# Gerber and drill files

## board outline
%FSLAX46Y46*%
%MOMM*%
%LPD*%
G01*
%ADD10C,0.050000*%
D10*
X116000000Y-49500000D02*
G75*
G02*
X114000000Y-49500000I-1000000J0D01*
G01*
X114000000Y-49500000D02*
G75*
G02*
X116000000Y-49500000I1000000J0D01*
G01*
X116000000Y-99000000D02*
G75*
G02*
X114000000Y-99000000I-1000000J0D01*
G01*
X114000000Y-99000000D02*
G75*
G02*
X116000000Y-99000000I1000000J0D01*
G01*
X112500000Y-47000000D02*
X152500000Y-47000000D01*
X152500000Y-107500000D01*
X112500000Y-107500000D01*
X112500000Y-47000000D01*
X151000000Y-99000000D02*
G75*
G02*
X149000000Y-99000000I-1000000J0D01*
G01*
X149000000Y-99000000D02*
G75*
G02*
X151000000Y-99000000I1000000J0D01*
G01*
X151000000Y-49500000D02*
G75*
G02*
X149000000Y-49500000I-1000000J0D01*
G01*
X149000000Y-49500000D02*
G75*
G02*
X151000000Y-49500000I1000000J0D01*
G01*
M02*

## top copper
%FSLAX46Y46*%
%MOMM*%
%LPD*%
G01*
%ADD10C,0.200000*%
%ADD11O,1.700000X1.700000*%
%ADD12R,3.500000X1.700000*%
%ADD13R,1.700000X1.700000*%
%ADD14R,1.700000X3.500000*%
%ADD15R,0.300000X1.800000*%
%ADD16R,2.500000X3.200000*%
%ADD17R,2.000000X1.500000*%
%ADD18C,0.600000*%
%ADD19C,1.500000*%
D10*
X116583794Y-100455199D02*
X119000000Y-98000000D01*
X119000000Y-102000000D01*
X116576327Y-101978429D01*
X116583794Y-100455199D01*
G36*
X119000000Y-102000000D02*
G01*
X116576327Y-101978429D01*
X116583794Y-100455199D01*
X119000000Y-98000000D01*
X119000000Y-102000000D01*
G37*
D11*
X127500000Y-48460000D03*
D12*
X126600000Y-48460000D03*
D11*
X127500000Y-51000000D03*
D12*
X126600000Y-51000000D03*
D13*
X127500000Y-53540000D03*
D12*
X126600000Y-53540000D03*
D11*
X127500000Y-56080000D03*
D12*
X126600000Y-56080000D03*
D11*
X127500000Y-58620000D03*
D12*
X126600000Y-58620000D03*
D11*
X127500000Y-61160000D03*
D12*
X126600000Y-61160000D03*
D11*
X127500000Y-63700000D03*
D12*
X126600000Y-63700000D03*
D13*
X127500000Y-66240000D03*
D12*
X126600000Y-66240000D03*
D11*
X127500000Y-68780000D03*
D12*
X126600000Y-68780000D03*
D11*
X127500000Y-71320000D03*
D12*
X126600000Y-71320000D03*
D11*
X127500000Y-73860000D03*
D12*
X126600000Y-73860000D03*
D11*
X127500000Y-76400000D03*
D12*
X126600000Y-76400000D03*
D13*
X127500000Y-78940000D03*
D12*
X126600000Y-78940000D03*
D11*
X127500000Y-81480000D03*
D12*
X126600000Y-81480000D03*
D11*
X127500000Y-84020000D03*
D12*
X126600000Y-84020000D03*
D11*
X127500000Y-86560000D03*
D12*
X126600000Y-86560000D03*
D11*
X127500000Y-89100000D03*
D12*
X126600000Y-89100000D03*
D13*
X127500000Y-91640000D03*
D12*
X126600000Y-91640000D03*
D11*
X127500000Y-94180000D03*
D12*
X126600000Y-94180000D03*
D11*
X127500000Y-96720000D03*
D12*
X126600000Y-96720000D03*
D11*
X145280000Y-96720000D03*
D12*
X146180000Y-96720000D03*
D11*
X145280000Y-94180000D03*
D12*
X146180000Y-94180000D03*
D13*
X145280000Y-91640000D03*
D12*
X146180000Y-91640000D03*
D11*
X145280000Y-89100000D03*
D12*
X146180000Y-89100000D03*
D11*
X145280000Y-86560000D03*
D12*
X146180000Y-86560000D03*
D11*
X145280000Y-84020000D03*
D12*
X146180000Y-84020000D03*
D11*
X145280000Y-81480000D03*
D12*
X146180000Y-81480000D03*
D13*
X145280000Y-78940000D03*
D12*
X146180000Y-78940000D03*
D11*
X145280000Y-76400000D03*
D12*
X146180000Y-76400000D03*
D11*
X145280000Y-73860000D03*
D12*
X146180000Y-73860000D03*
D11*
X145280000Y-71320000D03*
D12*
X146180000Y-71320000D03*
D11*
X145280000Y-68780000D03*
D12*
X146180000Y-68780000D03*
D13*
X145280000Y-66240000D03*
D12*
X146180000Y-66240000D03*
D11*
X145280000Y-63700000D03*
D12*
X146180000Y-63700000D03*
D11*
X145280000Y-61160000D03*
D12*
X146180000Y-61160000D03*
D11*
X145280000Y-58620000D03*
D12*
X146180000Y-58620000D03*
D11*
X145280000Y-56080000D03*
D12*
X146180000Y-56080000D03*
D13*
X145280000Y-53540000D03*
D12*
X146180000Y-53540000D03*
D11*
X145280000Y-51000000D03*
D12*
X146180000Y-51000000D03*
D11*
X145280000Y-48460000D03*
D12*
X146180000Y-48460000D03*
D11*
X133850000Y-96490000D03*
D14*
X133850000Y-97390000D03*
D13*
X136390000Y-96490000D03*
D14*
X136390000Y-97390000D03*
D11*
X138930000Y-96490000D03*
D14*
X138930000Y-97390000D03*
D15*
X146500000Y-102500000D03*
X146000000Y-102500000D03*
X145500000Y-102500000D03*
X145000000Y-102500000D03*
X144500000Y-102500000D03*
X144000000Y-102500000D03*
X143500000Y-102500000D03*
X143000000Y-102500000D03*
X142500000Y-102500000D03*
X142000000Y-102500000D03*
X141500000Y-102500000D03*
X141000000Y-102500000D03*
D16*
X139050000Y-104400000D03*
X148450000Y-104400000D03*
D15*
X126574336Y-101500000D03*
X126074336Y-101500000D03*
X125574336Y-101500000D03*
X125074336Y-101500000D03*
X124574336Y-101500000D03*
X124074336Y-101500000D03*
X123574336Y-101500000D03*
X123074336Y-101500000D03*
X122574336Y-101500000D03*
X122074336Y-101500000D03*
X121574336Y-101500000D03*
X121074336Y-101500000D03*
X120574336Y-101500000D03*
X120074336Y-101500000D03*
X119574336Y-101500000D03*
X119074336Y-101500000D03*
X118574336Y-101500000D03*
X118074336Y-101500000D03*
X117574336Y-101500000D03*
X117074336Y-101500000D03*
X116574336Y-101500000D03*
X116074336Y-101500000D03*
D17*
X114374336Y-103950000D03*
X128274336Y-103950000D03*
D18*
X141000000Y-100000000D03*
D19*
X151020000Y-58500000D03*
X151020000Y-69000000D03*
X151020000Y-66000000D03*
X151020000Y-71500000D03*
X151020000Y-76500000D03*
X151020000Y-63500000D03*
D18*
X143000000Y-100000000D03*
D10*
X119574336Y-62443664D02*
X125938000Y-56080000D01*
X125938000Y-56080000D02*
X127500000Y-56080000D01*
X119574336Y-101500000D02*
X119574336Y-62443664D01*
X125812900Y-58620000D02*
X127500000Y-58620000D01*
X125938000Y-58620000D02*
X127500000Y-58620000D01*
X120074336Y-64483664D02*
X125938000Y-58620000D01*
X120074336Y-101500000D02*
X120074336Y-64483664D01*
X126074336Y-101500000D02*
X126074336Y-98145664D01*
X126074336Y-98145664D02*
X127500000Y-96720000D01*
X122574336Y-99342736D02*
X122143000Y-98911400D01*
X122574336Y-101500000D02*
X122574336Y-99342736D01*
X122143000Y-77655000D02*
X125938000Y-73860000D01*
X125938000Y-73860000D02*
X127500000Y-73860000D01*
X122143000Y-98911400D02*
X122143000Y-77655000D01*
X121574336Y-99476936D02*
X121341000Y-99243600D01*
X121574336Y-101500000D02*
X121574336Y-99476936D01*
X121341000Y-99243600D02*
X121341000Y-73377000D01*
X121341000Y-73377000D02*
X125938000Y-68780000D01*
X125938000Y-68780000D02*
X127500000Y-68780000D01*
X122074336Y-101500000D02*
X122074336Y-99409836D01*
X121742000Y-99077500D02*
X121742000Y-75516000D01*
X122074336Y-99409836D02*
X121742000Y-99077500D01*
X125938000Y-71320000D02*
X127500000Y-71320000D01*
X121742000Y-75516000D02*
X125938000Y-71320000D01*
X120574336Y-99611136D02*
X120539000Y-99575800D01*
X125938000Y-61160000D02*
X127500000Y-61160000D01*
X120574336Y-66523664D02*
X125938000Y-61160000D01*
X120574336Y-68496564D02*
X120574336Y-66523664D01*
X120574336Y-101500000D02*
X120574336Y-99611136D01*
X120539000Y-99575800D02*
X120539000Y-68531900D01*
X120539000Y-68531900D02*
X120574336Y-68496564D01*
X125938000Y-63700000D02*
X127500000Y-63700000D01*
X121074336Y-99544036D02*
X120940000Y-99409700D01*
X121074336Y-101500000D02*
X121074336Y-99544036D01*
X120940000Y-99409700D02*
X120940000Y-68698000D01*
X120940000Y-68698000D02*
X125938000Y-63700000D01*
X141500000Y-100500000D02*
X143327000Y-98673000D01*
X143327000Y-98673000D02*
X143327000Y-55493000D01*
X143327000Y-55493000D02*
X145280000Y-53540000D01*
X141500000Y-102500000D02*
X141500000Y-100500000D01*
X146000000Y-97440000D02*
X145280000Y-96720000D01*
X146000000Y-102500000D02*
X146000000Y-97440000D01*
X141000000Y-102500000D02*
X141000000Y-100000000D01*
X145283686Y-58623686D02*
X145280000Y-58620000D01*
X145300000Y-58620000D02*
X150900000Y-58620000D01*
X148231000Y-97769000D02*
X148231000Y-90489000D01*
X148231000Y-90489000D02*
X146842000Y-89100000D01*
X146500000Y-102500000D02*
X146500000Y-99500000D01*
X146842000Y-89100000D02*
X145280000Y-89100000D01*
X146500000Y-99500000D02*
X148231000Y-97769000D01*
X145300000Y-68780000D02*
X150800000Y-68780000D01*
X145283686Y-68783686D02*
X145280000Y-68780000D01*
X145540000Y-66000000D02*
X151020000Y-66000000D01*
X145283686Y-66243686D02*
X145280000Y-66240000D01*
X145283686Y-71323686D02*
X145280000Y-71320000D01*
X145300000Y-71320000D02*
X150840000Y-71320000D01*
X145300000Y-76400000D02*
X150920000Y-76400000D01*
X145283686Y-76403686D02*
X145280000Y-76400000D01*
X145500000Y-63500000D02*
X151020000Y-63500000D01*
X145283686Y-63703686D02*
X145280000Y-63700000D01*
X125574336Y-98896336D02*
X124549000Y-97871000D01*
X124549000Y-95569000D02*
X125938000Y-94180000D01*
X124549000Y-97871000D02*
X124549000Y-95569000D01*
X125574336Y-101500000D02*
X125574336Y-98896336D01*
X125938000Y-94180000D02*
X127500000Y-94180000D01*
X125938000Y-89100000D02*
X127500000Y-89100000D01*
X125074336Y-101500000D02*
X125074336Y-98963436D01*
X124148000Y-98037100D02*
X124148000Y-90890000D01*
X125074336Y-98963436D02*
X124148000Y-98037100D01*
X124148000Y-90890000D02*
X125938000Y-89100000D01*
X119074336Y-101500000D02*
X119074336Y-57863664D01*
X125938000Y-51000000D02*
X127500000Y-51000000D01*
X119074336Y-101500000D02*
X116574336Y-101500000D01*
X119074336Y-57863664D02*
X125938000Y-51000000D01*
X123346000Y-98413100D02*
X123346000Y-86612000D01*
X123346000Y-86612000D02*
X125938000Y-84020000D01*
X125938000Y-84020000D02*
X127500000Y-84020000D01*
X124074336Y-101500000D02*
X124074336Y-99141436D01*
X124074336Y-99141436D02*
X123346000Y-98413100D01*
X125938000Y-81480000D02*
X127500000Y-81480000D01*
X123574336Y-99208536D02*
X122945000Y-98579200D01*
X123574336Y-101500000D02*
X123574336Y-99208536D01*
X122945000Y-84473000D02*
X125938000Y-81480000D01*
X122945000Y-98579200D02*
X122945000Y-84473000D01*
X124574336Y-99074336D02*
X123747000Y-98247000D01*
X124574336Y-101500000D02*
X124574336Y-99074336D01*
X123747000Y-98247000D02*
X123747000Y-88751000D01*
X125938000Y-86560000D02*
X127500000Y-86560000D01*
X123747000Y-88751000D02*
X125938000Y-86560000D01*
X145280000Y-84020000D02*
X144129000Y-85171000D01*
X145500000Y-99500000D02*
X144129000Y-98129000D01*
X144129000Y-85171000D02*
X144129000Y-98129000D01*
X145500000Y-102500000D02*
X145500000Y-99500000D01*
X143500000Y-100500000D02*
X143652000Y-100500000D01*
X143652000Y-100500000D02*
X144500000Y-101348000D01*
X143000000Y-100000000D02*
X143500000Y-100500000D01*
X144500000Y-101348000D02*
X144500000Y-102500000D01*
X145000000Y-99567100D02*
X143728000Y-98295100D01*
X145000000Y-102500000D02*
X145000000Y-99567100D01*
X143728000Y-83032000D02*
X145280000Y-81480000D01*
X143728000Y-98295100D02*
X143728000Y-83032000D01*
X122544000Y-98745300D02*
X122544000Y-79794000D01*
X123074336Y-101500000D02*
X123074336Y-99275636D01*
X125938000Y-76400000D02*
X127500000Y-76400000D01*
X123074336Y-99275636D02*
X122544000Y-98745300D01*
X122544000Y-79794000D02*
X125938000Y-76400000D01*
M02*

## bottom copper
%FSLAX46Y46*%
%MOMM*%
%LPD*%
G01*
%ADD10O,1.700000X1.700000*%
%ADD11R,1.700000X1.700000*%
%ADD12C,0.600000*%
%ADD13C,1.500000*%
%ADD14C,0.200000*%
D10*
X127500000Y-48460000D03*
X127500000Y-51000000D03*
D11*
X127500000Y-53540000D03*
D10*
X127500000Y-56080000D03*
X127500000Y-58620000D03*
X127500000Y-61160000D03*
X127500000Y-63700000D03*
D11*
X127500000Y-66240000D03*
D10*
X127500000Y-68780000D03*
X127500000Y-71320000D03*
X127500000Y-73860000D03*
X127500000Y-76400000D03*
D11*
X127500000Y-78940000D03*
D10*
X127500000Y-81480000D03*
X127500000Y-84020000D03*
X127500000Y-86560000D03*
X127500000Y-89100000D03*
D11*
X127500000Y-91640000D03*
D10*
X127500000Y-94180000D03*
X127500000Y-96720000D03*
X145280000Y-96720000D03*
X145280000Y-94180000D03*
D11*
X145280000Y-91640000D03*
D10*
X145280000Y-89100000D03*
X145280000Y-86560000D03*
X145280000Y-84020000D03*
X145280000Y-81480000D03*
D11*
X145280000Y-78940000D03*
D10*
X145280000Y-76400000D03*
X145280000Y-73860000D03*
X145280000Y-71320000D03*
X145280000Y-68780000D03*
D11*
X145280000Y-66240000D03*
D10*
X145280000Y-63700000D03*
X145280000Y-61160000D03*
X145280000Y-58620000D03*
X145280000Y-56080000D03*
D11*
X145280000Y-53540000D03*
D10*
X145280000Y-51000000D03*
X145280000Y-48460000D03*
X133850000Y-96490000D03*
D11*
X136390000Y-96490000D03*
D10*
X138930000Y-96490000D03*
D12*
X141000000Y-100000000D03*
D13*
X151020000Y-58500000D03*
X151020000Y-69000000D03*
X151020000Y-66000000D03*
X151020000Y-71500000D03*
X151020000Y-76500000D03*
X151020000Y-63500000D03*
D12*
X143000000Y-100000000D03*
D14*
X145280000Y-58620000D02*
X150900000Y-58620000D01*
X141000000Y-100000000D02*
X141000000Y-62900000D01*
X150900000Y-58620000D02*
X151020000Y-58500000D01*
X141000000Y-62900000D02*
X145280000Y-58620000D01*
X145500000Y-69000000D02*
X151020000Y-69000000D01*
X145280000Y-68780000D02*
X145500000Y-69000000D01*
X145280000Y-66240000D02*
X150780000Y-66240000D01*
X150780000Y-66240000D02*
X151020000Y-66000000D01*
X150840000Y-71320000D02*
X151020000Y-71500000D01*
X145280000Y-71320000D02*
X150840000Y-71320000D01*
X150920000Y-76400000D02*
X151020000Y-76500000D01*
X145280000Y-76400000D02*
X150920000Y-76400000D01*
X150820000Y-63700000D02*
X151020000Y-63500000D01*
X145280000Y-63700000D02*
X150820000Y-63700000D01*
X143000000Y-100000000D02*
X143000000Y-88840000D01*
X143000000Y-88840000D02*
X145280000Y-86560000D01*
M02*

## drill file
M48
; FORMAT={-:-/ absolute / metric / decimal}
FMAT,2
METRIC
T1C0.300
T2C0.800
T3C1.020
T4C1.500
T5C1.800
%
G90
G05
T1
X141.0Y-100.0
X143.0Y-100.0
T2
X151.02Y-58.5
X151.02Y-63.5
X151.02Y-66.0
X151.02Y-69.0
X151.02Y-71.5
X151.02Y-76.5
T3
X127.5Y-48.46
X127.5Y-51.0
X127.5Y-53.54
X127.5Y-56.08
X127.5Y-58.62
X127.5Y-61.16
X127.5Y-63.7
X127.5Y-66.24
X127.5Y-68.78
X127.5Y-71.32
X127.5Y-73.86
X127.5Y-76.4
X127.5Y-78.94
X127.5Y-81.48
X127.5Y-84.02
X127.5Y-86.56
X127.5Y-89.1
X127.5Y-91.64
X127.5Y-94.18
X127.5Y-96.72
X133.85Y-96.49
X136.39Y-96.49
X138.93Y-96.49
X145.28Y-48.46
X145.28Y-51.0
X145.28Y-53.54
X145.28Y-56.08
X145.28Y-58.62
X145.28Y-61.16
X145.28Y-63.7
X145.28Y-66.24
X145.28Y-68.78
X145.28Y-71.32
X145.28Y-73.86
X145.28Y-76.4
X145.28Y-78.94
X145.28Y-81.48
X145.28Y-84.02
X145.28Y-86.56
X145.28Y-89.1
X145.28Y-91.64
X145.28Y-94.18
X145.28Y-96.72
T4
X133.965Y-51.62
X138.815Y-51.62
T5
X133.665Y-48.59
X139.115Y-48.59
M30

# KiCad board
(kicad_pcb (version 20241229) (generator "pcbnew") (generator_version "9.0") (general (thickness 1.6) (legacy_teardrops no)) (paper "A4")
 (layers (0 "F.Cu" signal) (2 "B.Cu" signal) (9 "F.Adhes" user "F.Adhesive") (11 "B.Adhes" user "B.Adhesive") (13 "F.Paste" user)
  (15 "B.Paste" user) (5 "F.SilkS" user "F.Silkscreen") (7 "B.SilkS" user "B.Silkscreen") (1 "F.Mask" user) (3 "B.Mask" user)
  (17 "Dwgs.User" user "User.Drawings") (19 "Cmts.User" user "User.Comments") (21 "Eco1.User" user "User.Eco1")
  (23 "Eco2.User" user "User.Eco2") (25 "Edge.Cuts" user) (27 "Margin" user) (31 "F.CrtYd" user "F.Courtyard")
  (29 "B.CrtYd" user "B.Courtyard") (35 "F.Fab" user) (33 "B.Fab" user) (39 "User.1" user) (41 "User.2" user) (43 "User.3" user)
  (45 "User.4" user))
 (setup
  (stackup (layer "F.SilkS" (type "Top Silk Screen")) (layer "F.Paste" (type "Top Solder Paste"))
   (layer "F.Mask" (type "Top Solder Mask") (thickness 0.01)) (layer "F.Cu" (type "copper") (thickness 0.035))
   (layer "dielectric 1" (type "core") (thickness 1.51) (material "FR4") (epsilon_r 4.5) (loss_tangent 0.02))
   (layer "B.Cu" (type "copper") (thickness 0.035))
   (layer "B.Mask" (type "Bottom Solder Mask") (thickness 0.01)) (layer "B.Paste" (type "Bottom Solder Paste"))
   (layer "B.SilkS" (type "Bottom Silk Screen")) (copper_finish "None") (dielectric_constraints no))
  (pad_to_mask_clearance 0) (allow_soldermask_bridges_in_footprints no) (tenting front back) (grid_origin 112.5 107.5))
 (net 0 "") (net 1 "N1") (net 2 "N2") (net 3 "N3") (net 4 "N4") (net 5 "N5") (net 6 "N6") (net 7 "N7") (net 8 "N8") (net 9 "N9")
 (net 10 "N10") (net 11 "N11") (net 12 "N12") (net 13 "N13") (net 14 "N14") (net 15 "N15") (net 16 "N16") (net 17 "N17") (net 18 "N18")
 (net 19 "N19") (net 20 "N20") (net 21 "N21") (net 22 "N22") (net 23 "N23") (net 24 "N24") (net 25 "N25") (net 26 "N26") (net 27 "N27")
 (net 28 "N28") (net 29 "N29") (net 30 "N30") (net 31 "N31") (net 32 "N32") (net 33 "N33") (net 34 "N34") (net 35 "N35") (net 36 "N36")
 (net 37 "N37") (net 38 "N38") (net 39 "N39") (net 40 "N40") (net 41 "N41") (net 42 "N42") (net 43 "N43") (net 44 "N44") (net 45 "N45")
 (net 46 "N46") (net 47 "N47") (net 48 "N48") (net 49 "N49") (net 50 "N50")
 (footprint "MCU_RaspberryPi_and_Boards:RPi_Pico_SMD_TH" (layer "F.Cu") (at 136.39 72.59)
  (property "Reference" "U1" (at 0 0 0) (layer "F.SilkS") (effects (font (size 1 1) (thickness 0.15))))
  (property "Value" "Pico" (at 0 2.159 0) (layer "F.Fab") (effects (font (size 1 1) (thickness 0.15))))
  (pad "" np_thru_hole oval (at -2.725 -24) (size 1.8 1.8) (drill 1.8) (layers "*.Cu" "*.Mask"))
  (pad "" np_thru_hole oval (at -2.425 -20.97) (size 1.5 1.5) (drill 1.5) (layers "*.Cu" "*.Mask"))
  (pad "" np_thru_hole oval (at 2.425 -20.97) (size 1.5 1.5) (drill 1.5) (layers "*.Cu" "*.Mask"))
  (pad "" np_thru_hole oval (at 2.725 -24) (size 1.8 1.8) (drill 1.8) (layers "*.Cu" "*.Mask"))
  (pad "1" thru_hole oval (at -8.89 -24.13) (size 1.7 1.7) (drill 1.02) (layers "*.Cu" "*.Mask") (remove_unused_layers no) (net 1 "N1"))
  (pad "1" smd rect (at -8.89 -24.13) (size 3.5 1.7) (drill (offset -0.9 0)) (layers "F.Cu" "F.Mask") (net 1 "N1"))
  (pad "2" thru_hole oval (at -8.89 -21.59) (size 1.7 1.7) (drill 1.02) (layers "*.Cu" "*.Mask") (remove_unused_layers no) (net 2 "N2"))
  (pad "2" smd rect (at -8.89 -21.59) (size 3.5 1.7) (drill (offset -0.9 0)) (layers "F.Cu" "F.Mask") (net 2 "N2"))
  (pad "3" thru_hole rect (at -8.89 -19.05) (size 1.7 1.7) (drill 1.02) (layers "*.Cu" "*.Mask") (remove_unused_layers no) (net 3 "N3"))
  (pad "3" smd rect (at -8.89 -19.05) (size 3.5 1.7) (drill (offset -0.9 0)) (layers "F.Cu" "F.Mask") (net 3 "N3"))
  (pad "4" thru_hole oval (at -8.89 -16.51) (size 1.7 1.7) (drill 1.02) (layers "*.Cu" "*.Mask") (remove_unused_layers no) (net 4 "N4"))
  (pad "4" smd rect (at -8.89 -16.51) (size 3.5 1.7) (drill (offset -0.9 0)) (layers "F.Cu" "F.Mask") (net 4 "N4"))
  (pad "5" thru_hole oval (at -8.89 -13.97) (size 1.7 1.7) (drill 1.02) (layers "*.Cu" "*.Mask") (remove_unused_layers no) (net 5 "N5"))
  (pad "5" smd rect (at -8.89 -13.97) (size 3.5 1.7) (drill (offset -0.9 0)) (layers "F.Cu" "F.Mask") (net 5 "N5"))
  (pad "6" thru_hole oval (at -8.89 -11.43) (size 1.7 1.7) (drill 1.02) (layers "*.Cu" "*.Mask") (remove_unused_layers no) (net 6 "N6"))
  (pad "6" smd rect (at -8.89 -11.43) (size 3.5 1.7) (drill (offset -0.9 0)) (layers "F.Cu" "F.Mask") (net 6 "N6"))
  (pad "7" thru_hole oval (at -8.89 -8.89) (size 1.7 1.7) (drill 1.02) (layers "*.Cu" "*.Mask") (remove_unused_layers no) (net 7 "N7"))
  (pad "7" smd rect (at -8.89 -8.89) (size 3.5 1.7) (drill (offset -0.9 0)) (layers "F.Cu" "F.Mask") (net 7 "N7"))
  (pad "8" thru_hole rect (at -8.89 -6.35) (size 1.7 1.7) (drill 1.02) (layers "*.Cu" "*.Mask") (remove_unused_layers no) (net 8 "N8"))
  (pad "8" smd rect (at -8.89 -6.35) (size 3.5 1.7) (drill (offset -0.9 0)) (layers "F.Cu" "F.Mask") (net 8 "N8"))
  (pad "9" thru_hole oval (at -8.89 -3.81) (size 1.7 1.7) (drill 1.02) (layers "*.Cu" "*.Mask") (remove_unused_layers no) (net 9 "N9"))
  (pad "9" smd rect (at -8.89 -3.81) (size 3.5 1.7) (drill (offset -0.9 0)) (layers "F.Cu" "F.Mask") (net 9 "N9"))
  (pad "10" thru_hole oval (at -8.89 -1.27) (size 1.7 1.7) (drill 1.02) (layers "*.Cu" "*.Mask") (remove_unused_layers no) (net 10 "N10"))
  (pad "10" smd rect (at -8.89 -1.27) (size 3.5 1.7) (drill (offset -0.9 0)) (layers "F.Cu" "F.Mask") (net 10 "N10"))
  (pad "11" thru_hole oval (at -8.89 1.27) (size 1.7 1.7) (drill 1.02) (layers "*.Cu" "*.Mask") (remove_unused_layers no) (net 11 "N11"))
  (pad "11" smd rect (at -8.89 1.27) (size 3.5 1.7) (drill (offset -0.9 0)) (layers "F.Cu" "F.Mask") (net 11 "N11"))
  (pad "12" thru_hole oval (at -8.89 3.81) (size 1.7 1.7) (drill 1.02) (layers "*.Cu" "*.Mask") (remove_unused_layers no) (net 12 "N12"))
  (pad "12" smd rect (at -8.89 3.81) (size 3.5 1.7) (drill (offset -0.9 0)) (layers "F.Cu" "F.Mask") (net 12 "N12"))
  (pad "13" thru_hole rect (at -8.89 6.35) (size 1.7 1.7) (drill 1.02) (layers "*.Cu" "*.Mask") (remove_unused_layers no) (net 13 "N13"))
  (pad "13" smd rect (at -8.89 6.35) (size 3.5 1.7) (drill (offset -0.9 0)) (layers "F.Cu" "F.Mask") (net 13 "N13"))
  (pad "14" thru_hole oval (at -8.89 8.89) (size 1.7 1.7) (drill 1.02) (layers "*.Cu" "*.Mask") (remove_unused_layers no) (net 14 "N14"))
  (pad "14" smd rect (at -8.89 8.89) (size 3.5 1.7) (drill (offset -0.9 0)) (layers "F.Cu" "F.Mask") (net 14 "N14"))
  (pad "15" thru_hole oval (at -8.89 11.43) (size 1.7 1.7) (drill 1.02) (layers "*.Cu" "*.Mask") (remove_unused_layers no) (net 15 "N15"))
  (pad "15" smd rect (at -8.89 11.43) (size 3.5 1.7) (drill (offset -0.9 0)) (layers "F.Cu" "F.Mask") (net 15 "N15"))
  (pad "16" thru_hole oval (at -8.89 13.97) (size 1.7 1.7) (drill 1.02) (layers "*.Cu" "*.Mask") (remove_unused_layers no) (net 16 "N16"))
  (pad "16" smd rect (at -8.89 13.97) (size 3.5 1.7) (drill (offset -0.9 0)) (layers "F.Cu" "F.Mask") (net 16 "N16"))
  (pad "17" thru_hole oval (at -8.89 16.51) (size 1.7 1.7) (drill 1.02) (layers "*.Cu" "*.Mask") (remove_unused_layers no) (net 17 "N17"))
  (pad "17" smd rect (at -8.89 16.51) (size 3.5 1.7) (drill (offset -0.9 0)) (layers "F.Cu" "F.Mask") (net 17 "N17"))
  (pad "18" thru_hole rect (at -8.89 19.05) (size 1.7 1.7) (drill 1.02) (layers "*.Cu" "*.Mask") (remove_unused_layers no) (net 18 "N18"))
  (pad "18" smd rect (at -8.89 19.05) (size 3.5 1.7) (drill (offset -0.9 0)) (layers "F.Cu" "F.Mask") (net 18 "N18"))
  (pad "19" thru_hole oval (at -8.89 21.59) (size 1.7 1.7) (drill 1.02) (layers "*.Cu" "*.Mask") (remove_unused_layers no) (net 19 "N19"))
  (pad "19" smd rect (at -8.89 21.59) (size 3.5 1.7) (drill (offset -0.9 0)) (layers "F.Cu" "F.Mask") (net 19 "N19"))
  (pad "20" thru_hole oval (at -8.89 24.13) (size 1.7 1.7) (drill 1.02) (layers "*.Cu" "*.Mask") (remove_unused_layers no) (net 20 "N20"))
  (pad "20" smd rect (at -8.89 24.13) (size 3.5 1.7) (drill (offset -0.9 0)) (layers "F.Cu" "F.Mask") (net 20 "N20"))
  (pad "21" thru_hole oval (at 8.89 24.13) (size 1.7 1.7) (drill 1.02) (layers "*.Cu" "*.Mask") (remove_unused_layers no) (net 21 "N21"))
  (pad "21" smd rect (at 8.89 24.13) (size 3.5 1.7) (drill (offset 0.9 0)) (layers "F.Cu" "F.Mask") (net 21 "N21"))
  (pad "22" thru_hole oval (at 8.89 21.59) (size 1.7 1.7) (drill 1.02) (layers "*.Cu" "*.Mask") (remove_unused_layers no) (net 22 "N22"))
  (pad "22" smd rect (at 8.89 21.59) (size 3.5 1.7) (drill (offset 0.9 0)) (layers "F.Cu" "F.Mask") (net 22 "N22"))
  (pad "23" thru_hole rect (at 8.89 19.05) (size 1.7 1.7) (drill 1.02) (layers "*.Cu" "*.Mask") (remove_unused_layers no) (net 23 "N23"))
  (pad "23" smd rect (at 8.89 19.05) (size 3.5 1.7) (drill (offset 0.9 0)) (layers "F.Cu" "F.Mask") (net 23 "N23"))
  (pad "24" thru_hole oval (at 8.89 16.51) (size 1.7 1.7) (drill 1.02) (layers "*.Cu" "*.Mask") (remove_unused_layers no) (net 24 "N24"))
  (pad "24" smd rect (at 8.89 16.51) (size 3.5 1.7) (drill (offset 0.9 0)) (layers "F.Cu" "F.Mask") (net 24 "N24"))
  (pad "25" thru_hole oval (at 8.89 13.97) (size 1.7 1.7) (drill 1.02) (layers "*.Cu" "*.Mask") (remove_unused_layers no) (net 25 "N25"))
  (pad "25" smd rect (at 8.89 13.97) (size 3.5 1.7) (drill (offset 0.9 0)) (layers "F.Cu" "F.Mask") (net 25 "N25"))
  (pad "26" thru_hole oval (at 8.89 11.43) (size 1.7 1.7) (drill 1.02) (layers "*.Cu" "*.Mask") (remove_unused_layers no) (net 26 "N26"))
  (pad "26" smd rect (at 8.89 11.43) (size 3.5 1.7) (drill (offset 0.9 0)) (layers "F.Cu" "F.Mask") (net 26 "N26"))
  (pad "27" thru_hole oval (at 8.89 8.89) (size 1.7 1.7) (drill 1.02) (layers "*.Cu" "*.Mask") (remove_unused_layers no) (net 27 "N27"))
  (pad "27" smd rect (at 8.89 8.89) (size 3.5 1.7) (drill (offset 0.9 0)) (layers "F.Cu" "F.Mask") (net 27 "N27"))
  (pad "28" thru_hole rect (at 8.89 6.35) (size 1.7 1.7) (drill 1.02) (layers "*.Cu" "*.Mask") (remove_unused_layers no) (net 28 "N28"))
  (pad "28" smd rect (at 8.89 6.35) (size 3.5 1.7) (drill (offset 0.9 0)) (layers "F.Cu" "F.Mask") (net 28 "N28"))
  (pad "29" thru_hole oval (at 8.89 3.81) (size 1.7 1.7) (drill 1.02) (layers "*.Cu" "*.Mask") (remove_unused_layers no) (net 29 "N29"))
  (pad "29" smd rect (at 8.89 3.81) (size 3.5 1.7) (drill (offset 0.9 0)) (layers "F.Cu" "F.Mask") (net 29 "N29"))
  (pad "30" thru_hole oval (at 8.89 1.27) (size 1.7 1.7) (drill 1.02) (layers "*.Cu" "*.Mask") (remove_unused_layers no) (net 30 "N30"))
  (pad "30" smd rect (at 8.89 1.27) (size 3.5 1.7) (drill (offset 0.9 0)) (layers "F.Cu" "F.Mask") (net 30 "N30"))
  (pad "31" thru_hole oval (at 8.89 -1.27) (size 1.7 1.7) (drill 1.02) (layers "*.Cu" "*.Mask") (remove_unused_layers no) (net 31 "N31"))
  (pad "31" smd rect (at 8.89 -1.27) (size 3.5 1.7) (drill (offset 0.9 0)) (layers "F.Cu" "F.Mask") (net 31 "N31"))
  (pad "32" thru_hole oval (at 8.89 -3.81) (size 1.7 1.7) (drill 1.02) (layers "*.Cu" "*.Mask") (remove_unused_layers no) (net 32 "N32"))
  (pad "32" smd rect (at 8.89 -3.81) (size 3.5 1.7) (drill (offset 0.9 0)) (layers "F.Cu" "F.Mask") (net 32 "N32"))
  (pad "33" thru_hole rect (at 8.89 -6.35) (size 1.7 1.7) (drill 1.02) (layers "*.Cu" "*.Mask") (remove_unused_layers no) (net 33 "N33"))
  (pad "33" smd rect (at 8.89 -6.35) (size 3.5 1.7) (drill (offset 0.9 0)) (layers "F.Cu" "F.Mask") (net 33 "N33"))
  (pad "34" thru_hole oval (at 8.89 -8.89) (size 1.7 1.7) (drill 1.02) (layers "*.Cu" "*.Mask") (remove_unused_layers no) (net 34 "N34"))
  (pad "34" smd rect (at 8.89 -8.89) (size 3.5 1.7) (drill (offset 0.9 0)) (layers "F.Cu" "F.Mask") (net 34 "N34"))
  (pad "35" thru_hole oval (at 8.89 -11.43) (size 1.7 1.7) (drill 1.02) (layers "*.Cu" "*.Mask") (remove_unused_layers no) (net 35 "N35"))
  (pad "35" smd rect (at 8.89 -11.43) (size 3.5 1.7) (drill (offset 0.9 0)) (layers "F.Cu" "F.Mask") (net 35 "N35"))
  (pad "36" thru_hole oval (at 8.89 -13.97) (size 1.7 1.7) (drill 1.02) (layers "*.Cu" "*.Mask") (remove_unused_layers no) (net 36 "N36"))
  (pad "36" smd rect (at 8.89 -13.97) (size 3.5 1.7) (drill (offset 0.9 0)) (layers "F.Cu" "F.Mask") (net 36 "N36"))
  (pad "37" thru_hole oval (at 8.89 -16.51) (size 1.7 1.7) (drill 1.02) (layers "*.Cu" "*.Mask") (remove_unused_layers no) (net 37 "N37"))
  (pad "37" smd rect (at 8.89 -16.51) (size 3.5 1.7) (drill (offset 0.9 0)) (layers "F.Cu" "F.Mask") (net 37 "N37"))
  (pad "38" thru_hole rect (at 8.89 -19.05) (size 1.7 1.7) (drill 1.02) (layers "*.Cu" "*.Mask") (remove_unused_layers no) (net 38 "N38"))
  (pad "38" smd rect (at 8.89 -19.05) (size 3.5 1.7) (drill (offset 0.9 0)) (layers "F.Cu" "F.Mask") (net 38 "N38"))
  (pad "39" thru_hole oval (at 8.89 -21.59) (size 1.7 1.7) (drill 1.02) (layers "*.Cu" "*.Mask") (remove_unused_layers no) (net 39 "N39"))
  (pad "39" smd rect (at 8.89 -21.59) (size 3.5 1.7) (drill (offset 0.9 0)) (layers "F.Cu" "F.Mask") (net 39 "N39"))
  (pad "40" thru_hole oval (at 8.89 -24.13) (size 1.7 1.7) (drill 1.02) (layers "*.Cu" "*.Mask") (remove_unused_layers no) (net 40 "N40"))
  (pad "40" smd rect (at 8.89 -24.13) (size 3.5 1.7) (drill (offset 0.9 0)) (layers "F.Cu" "F.Mask") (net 40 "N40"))
  (pad "41" thru_hole oval (at -2.54 23.9) (size 1.7 1.7) (drill 1.02) (layers "*.Cu" "*.Mask") (remove_unused_layers no) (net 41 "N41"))
  (pad "41" smd rect (at -2.54 23.9 90) (size 3.5 1.7) (drill (offset -0.9 0)) (layers "F.Cu" "F.Mask") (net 41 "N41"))
  (pad "42" thru_hole rect (at 0 23.9) (size 1.7 1.7) (drill 1.02) (layers "*.Cu" "*.Mask") (remove_unused_layers no) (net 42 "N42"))
  (pad "42" smd rect (at 0 23.9 90) (size 3.5 1.7) (drill (offset -0.9 0)) (layers "F.Cu" "F.Mask") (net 42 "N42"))
  (pad "43" thru_hole oval (at 2.54 23.9) (size 1.7 1.7) (drill 1.02) (layers "*.Cu" "*.Mask") (remove_unused_layers no) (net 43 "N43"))
  (pad "43" smd rect (at 2.54 23.9 90) (size 3.5 1.7) (drill (offset -0.9 0)) (layers "F.Cu" "F.Mask") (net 43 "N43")))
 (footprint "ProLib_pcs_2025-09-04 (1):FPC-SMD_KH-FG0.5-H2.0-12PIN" (layer "F.Cu") (at 143.75 103.45 180)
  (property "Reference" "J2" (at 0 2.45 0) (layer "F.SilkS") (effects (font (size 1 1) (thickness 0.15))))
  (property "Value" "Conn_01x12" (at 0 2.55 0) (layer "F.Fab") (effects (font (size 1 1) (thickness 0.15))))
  (pad "1" smd rect (at -2.75 0.95 180) (size 0.3 1.8) (layers "F.Cu" "F.Mask" "F.Paste") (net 24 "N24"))
  (pad "2" smd rect (at -2.25 0.95 180) (size 0.3 1.8) (layers "F.Cu" "F.Mask" "F.Paste") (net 21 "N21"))
  (pad "3" smd rect (at -1.75 0.95 180) (size 0.3 1.8) (layers "F.Cu" "F.Mask" "F.Paste") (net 26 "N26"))
  (pad "4" smd rect (at -1.25 0.95 180) (size 0.3 1.8) (layers "F.Cu" "F.Mask" "F.Paste") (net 27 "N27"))
  (pad "5" smd rect (at -0.75 0.95 180) (size 0.3 1.8) (layers "F.Cu" "F.Mask" "F.Paste") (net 25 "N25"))
  (pad "6" smd rect (at -0.25 0.95 180) (size 0.3 1.8) (layers "F.Cu" "F.Mask" "F.Paste") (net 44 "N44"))
  (pad "7" smd rect (at 0.25 0.95 180) (size 0.3 1.8) (layers "F.Cu" "F.Mask" "F.Paste") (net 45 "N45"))
  (pad "8" smd rect (at 0.75 0.95 180) (size 0.3 1.8) (layers "F.Cu" "F.Mask" "F.Paste") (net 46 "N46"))
  (pad "9" smd rect (at 1.25 0.95 180) (size 0.3 1.8) (layers "F.Cu" "F.Mask" "F.Paste") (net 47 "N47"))
  (pad "10" smd rect (at 1.75 0.95 180) (size 0.3 1.8) (layers "F.Cu" "F.Mask" "F.Paste") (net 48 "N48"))
  (pad "11" smd rect (at 2.25 0.95 180) (size 0.3 1.8) (layers "F.Cu" "F.Mask" "F.Paste") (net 38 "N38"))
  (pad "12" smd rect (at 2.75 0.95 180) (size 0.3 1.8) (layers "F.Cu" "F.Mask" "F.Paste") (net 36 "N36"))
  (pad "13" smd rect (at 4.7 -0.95 180) (size 2.5 3.2) (layers "F.Cu" "F.Mask" "F.Paste"))
  (pad "14" smd rect (at -4.7 -0.95 180) (size 2.5 3.2) (layers "F.Cu" "F.Mask" "F.Paste")))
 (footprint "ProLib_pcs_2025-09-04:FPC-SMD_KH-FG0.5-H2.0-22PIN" (layer "F.Cu") (at 121.324336 102.725)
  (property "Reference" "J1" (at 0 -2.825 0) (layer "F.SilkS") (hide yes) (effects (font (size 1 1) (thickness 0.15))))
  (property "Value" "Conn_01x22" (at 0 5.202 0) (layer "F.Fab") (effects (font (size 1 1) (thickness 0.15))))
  (pad "1" smd rect (at 5.25 -1.225 180) (size 0.3 1.8) (layers "F.Cu" "F.Mask" "F.Paste") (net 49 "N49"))
  (pad "2" smd rect (at 4.75 -1.225 180) (size 0.3 1.8) (layers "F.Cu" "F.Mask" "F.Paste") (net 20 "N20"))
  (pad "3" smd rect (at 4.25 -1.225 180) (size 0.3 1.8) (layers "F.Cu" "F.Mask" "F.Paste") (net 19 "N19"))
  (pad "4" smd rect (at 3.75 -1.225 180) (size 0.3 1.8) (layers "F.Cu" "F.Mask" "F.Paste") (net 17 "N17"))
  (pad "5" smd rect (at 3.25 -1.225 180) (size 0.3 1.8) (layers "F.Cu" "F.Mask" "F.Paste") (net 16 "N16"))
  (pad "6" smd rect (at 2.75 -1.225 180) (size 0.3 1.8) (layers "F.Cu" "F.Mask" "F.Paste") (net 15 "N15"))
  (pad "7" smd rect (at 2.25 -1.225 180) (size 0.3 1.8) (layers "F.Cu" "F.Mask" "F.Paste") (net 14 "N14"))
  (pad "8" smd rect (at 1.75 -1.225 180) (size 0.3 1.8) (layers "F.Cu" "F.Mask" "F.Paste") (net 12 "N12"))
  (pad "9" smd rect (at 1.25 -1.225 180) (size 0.3 1.8) (layers "F.Cu" "F.Mask" "F.Paste") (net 11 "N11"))
  (pad "10" smd rect (at 0.75 -1.225 180) (size 0.3 1.8) (layers "F.Cu" "F.Mask" "F.Paste") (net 10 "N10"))
  (pad "11" smd rect (at 0.25 -1.225 180) (size 0.3 1.8) (layers "F.Cu" "F.Mask" "F.Paste") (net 9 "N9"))
  (pad "12" smd rect (at -0.25 -1.225 180) (size 0.3 1.8) (layers "F.Cu" "F.Mask" "F.Paste") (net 7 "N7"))
  (pad "13" smd rect (at -0.75 -1.225 180) (size 0.3 1.8) (layers "F.Cu" "F.Mask" "F.Paste") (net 6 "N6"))
  (pad "14" smd rect (at -1.25 -1.225 180) (size 0.3 1.8) (layers "F.Cu" "F.Mask" "F.Paste") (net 5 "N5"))
  (pad "15" smd rect (at -1.75 -1.225 180) (size 0.3 1.8) (layers "F.Cu" "F.Mask" "F.Paste") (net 4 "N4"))
  (pad "16" smd rect (at -2.25 -1.225 180) (size 0.3 1.8) (layers "F.Cu" "F.Mask" "F.Paste") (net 2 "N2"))
  (pad "17" smd rect (at -2.75 -1.225 180) (size 0.3 1.8) (layers "F.Cu" "F.Mask" "F.Paste") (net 2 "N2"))
  (pad "18" smd rect (at -3.25 -1.225 180) (size 0.3 1.8) (layers "F.Cu" "F.Mask" "F.Paste") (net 2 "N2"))
  (pad "19" smd rect (at -3.75 -1.225 180) (size 0.3 1.8) (layers "F.Cu" "F.Mask" "F.Paste") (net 2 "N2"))
  (pad "20" smd rect (at -4.25 -1.225 180) (size 0.3 1.8) (layers "F.Cu" "F.Mask" "F.Paste") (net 2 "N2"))
  (pad "21" smd rect (at -4.75 -1.225 180) (size 0.3 1.8) (layers "F.Cu" "F.Mask" "F.Paste") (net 2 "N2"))
  (pad "22" smd rect (at -5.25 -1.225 180) (size 0.3 1.8) (layers "F.Cu" "F.Mask" "F.Paste") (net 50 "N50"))
  (pad "23" smd rect (at -6.95 1.225 180) (size 2 1.5) (layers "F.Cu" "F.Mask" "F.Paste"))
  (pad "24" smd rect (at 6.95 1.225 180) (size 2 1.5) (layers "F.Cu" "F.Mask" "F.Paste")))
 (gr_poly
  (pts (xy 116.583794 100.455199) (xy 119 98) (xy 119 102) (xy 116.576327 101.978429)) (stroke (width 0.2) (type solid)) (fill yes)
  (layer "F.Cu") (net 2))
 (gr_circle (center 115 49.5) (end 116 49.5) (stroke (width 0.05) (type default)) (fill no) (layer "Edge.Cuts"))
 (gr_circle (center 115 99) (end 116 99) (stroke (width 0.05) (type default)) (fill no) (layer "Edge.Cuts"))
 (gr_rect (start 112.5 47) (end 152.5 107.5) (stroke (width 0.05) (type default)) (fill no) (layer "Edge.Cuts"))
 (gr_circle (center 150 99) (end 151 99) (stroke (width 0.05) (type default)) (fill no) (layer "Edge.Cuts"))
 (gr_circle (center 150 49.5) (end 151 49.5) (stroke (width 0.05) (type default)) (fill no) (layer "Edge.Cuts"))
 (segment (start 119.574336 62.443664) (end 125.938 56.08) (width 0.2) (layer "F.Cu") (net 4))
 (segment (start 125.938 56.08) (end 127.5 56.08) (width 0.2) (layer "F.Cu") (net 4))
 (segment (start 119.574336 101.5) (end 119.574336 62.443664) (width 0.2) (layer "F.Cu") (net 4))
 (segment (start 125.8129 58.62) (end 127.5 58.62) (width 0.2) (layer "F.Cu") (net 5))
 (segment (start 125.938 58.62) (end 127.5 58.62) (width 0.2) (layer "F.Cu") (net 5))
 (segment (start 120.074336 64.483664) (end 125.938 58.62) (width 0.2) (layer "F.Cu") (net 5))
 (segment (start 120.074336 101.5) (end 120.074336 64.483664) (width 0.2) (layer "F.Cu") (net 5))
 (segment (start 126.074336 101.5) (end 126.074336 98.145664) (width 0.2) (layer "F.Cu") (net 20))
 (segment (start 126.074336 98.145664) (end 127.5 96.72) (width 0.2) (layer "F.Cu") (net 20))
 (segment (start 122.574336 99.342736) (end 122.143 98.9114) (width 0.2) (layer "F.Cu") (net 11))
 (segment (start 122.574336 101.5) (end 122.574336 99.342736) (width 0.2) (layer "F.Cu") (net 11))
 (segment (start 122.143 77.655) (end 125.938 73.86) (width 0.2) (layer "F.Cu") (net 11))
 (segment (start 125.938 73.86) (end 127.5 73.86) (width 0.2) (layer "F.Cu") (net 11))
 (segment (start 122.143 98.9114) (end 122.143 77.655) (width 0.2) (layer "F.Cu") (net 11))
 (segment (start 121.574336 99.476936) (end 121.341 99.2436) (width 0.2) (layer "F.Cu") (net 9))
 (segment (start 121.574336 101.5) (end 121.574336 99.476936) (width 0.2) (layer "F.Cu") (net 9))
 (segment (start 121.341 99.2436) (end 121.341 73.377) (width 0.2) (layer "F.Cu") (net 9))
 (segment (start 121.341 73.377) (end 125.938 68.78) (width 0.2) (layer "F.Cu") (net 9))
 (segment (start 125.938 68.78) (end 127.5 68.78) (width 0.2) (layer "F.Cu") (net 9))
 (segment (start 122.074336 101.5) (end 122.074336 99.409836) (width 0.2) (layer "F.Cu") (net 10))
 (segment (start 121.742 99.0775) (end 121.742 75.516) (width 0.2) (layer "F.Cu") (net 10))
 (segment (start 122.074336 99.409836) (end 121.742 99.0775) (width 0.2) (layer "F.Cu") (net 10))
 (segment (start 125.938 71.32) (end 127.5 71.32) (width 0.2) (layer "F.Cu") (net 10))
 (segment (start 121.742 75.516) (end 125.938 71.32) (width 0.2) (layer "F.Cu") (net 10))
 (segment (start 120.574336 99.611136) (end 120.539 99.5758) (width 0.2) (layer "F.Cu") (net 6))
 (segment (start 125.938 61.16) (end 127.5 61.16) (width 0.2) (layer "F.Cu") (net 6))
 (segment (start 120.574336 66.523664) (end 125.938 61.16) (width 0.2) (layer "F.Cu") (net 6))
 (segment (start 120.574336 68.496564) (end 120.574336 66.523664) (width 0.2) (layer "F.Cu") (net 6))
 (segment (start 120.574336 101.5) (end 120.574336 99.611136) (width 0.2) (layer "F.Cu") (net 6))
 (segment (start 120.539 99.5758) (end 120.539 68.5319) (width 0.2) (layer "F.Cu") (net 6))
 (segment (start 120.539 68.5319) (end 120.574336 68.496564) (width 0.2) (layer "F.Cu") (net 6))
 (segment (start 125.938 63.7) (end 127.5 63.7) (width 0.2) (layer "F.Cu") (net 7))
 (segment (start 121.074336 99.544036) (end 120.94 99.4097) (width 0.2) (layer "F.Cu") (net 7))
 (segment (start 121.074336 101.5) (end 121.074336 99.544036) (width 0.2) (layer "F.Cu") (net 7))
 (segment (start 120.94 99.4097) (end 120.94 68.698) (width 0.2) (layer "F.Cu") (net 7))
 (segment (start 120.94 68.698) (end 125.938 63.7) (width 0.2) (layer "F.Cu") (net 7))
 (segment (start 141.5 100.5) (end 143.327 98.673) (width 0.2) (layer "F.Cu") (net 38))
 (segment (start 143.327 98.673) (end 143.327 55.493) (width 0.2) (layer "F.Cu") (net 38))
 (segment (start 143.327 55.493) (end 145.28 53.54) (width 0.2) (layer "F.Cu") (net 38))
 (segment (start 141.5 102.5) (end 141.5 100.5) (width 0.2) (layer "F.Cu") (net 38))
 (segment (start 146 97.44) (end 145.28 96.72) (width 0.2) (layer "F.Cu") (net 21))
 (segment (start 146 102.5) (end 146 97.44) (width 0.2) (layer "F.Cu") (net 21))
 (segment (start 141 102.5) (end 141 100) (width 0.2) (layer "F.Cu") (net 36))
 (segment (start 145.283686 58.623686) (end 145.28 58.62) (width 0.2) (layer "F.Cu") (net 36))
 (segment (start 145.3 58.62) (end 150.9 58.62) (width 0.2) (layer "F.Cu") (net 36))
 (via (at 141 100) (size 0.6) (drill 0.3) (layers "F.Cu" "B.Cu") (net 36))
 (via (at 151.02 58.5) (size 1.5) (drill 0.8) (layers "F.Cu" "B.Cu") (tenting none) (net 36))
 (segment (start 145.28 58.62) (end 150.9 58.62) (width 0.2) (layer "B.Cu") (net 36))
 (segment (start 141 100) (end 141 62.9) (width 0.2) (layer "B.Cu") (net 36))
 (segment (start 150.9 58.62) (end 151.02 58.5) (width 0.2) (layer "B.Cu") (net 36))
 (segment (start 141 62.9) (end 145.28 58.62) (width 0.2) (layer "B.Cu") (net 36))
 (segment (start 148.231 97.769) (end 148.231 90.489) (width 0.2) (layer "F.Cu") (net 24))
 (segment (start 148.231 90.489) (end 146.842 89.1) (width 0.2) (layer "F.Cu") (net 24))
 (segment (start 146.5 102.5) (end 146.5 99.5) (width 0.2) (layer "F.Cu") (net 24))
 (segment (start 146.842 89.1) (end 145.28 89.1) (width 0.2) (layer "F.Cu") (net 24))
 (segment (start 146.5 99.5) (end 148.231 97.769) (width 0.2) (layer "F.Cu") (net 24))
 (segment (start 145.3 68.78) (end 150.8 68.78) (width 0.2) (layer "F.Cu") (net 32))
 (segment (start 145.283686 68.783686) (end 145.28 68.78) (width 0.2) (layer "F.Cu") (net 32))
 (via (at 151.02 69) (size 1.5) (drill 0.8) (layers "F.Cu" "B.Cu") (tenting none) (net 32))
 (segment (start 145.5 69) (end 151.02 69) (width 0.2) (layer "B.Cu") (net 32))
 (segment (start 145.28 68.78) (end 145.5 69) (width 0.2) (layer "B.Cu") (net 32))
 (segment (start 145.54 66) (end 151.02 66) (width 0.2) (layer "F.Cu") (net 33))
 (segment (start 145.283686 66.243686) (end 145.28 66.24) (width 0.2) (layer "F.Cu") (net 33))
 (via (at 151.02 66) (size 1.5) (drill 0.8) (layers "F.Cu" "B.Cu") (tenting none) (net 33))
 (segment (start 145.28 66.24) (end 150.78 66.24) (width 0.2) (layer "B.Cu") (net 33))
 (segment (start 150.78 66.24) (end 151.02 66) (width 0.2) (layer "B.Cu") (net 33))
 (segment (start 145.283686 71.323686) (end 145.28 71.32) (width 0.2) (layer "F.Cu") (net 31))
 (segment (start 145.3 71.32) (end 150.84 71.32) (width 0.2) (layer "F.Cu") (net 31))
 (via (at 151.02 71.5) (size 1.5) (drill 0.8) (layers "F.Cu" "B.Cu") (tenting none) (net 31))
 (segment (start 150.84 71.32) (end 151.02 71.5) (width 0.2) (layer "B.Cu") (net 31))
 (segment (start 145.28 71.32) (end 150.84 71.32) (width 0.2) (layer "B.Cu") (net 31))
 (segment (start 145.3 76.4) (end 150.92 76.4) (width 0.2) (layer "F.Cu") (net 29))
 (segment (start 145.283686 76.403686) (end 145.28 76.4) (width 0.2) (layer "F.Cu") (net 29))
 (via (at 151.02 76.5) (size 1.5) (drill 0.8) (layers "F.Cu" "B.Cu") (tenting none) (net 29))
 (segment (start 150.92 76.4) (end 151.02 76.5) (width 0.2) (layer "B.Cu") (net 29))
 (segment (start 145.28 76.4) (end 150.92 76.4) (width 0.2) (layer "B.Cu") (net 29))
 (segment (start 145.5 63.5) (end 151.02 63.5) (width 0.2) (layer "F.Cu") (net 34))
 (segment (start 145.283686 63.703686) (end 145.28 63.7) (width 0.2) (layer "F.Cu") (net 34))
 (via (at 151.02 63.5) (size 1.5) (drill 0.8) (layers "F.Cu" "B.Cu") (tenting none) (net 34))
 (segment (start 150.82 63.7) (end 151.02 63.5) (width 0.2) (layer "B.Cu") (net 34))
 (segment (start 145.28 63.7) (end 150.82 63.7) (width 0.2) (layer "B.Cu") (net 34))
 (segment (start 125.574336 98.896336) (end 124.549 97.871) (width 0.2) (layer "F.Cu") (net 19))
 (segment (start 124.549 95.569) (end 125.938 94.18) (width 0.2) (layer "F.Cu") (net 19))
 (segment (start 124.549 97.871) (end 124.549 95.569) (width 0.2) (layer "F.Cu") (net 19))
 (segment (start 125.574336 101.5) (end 125.574336 98.896336) (width 0.2) (layer "F.Cu") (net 19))
 (segment (start 125.938 94.18) (end 127.5 94.18) (width 0.2) (layer "F.Cu") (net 19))
 (segment (start 125.938 89.1) (end 127.5 89.1) (width 0.2) (layer "F.Cu") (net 17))
 (segment (start 125.074336 101.5) (end 125.074336 98.963436) (width 0.2) (layer "F.Cu") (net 17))
 (segment (start 124.148 98.0371) (end 124.148 90.89) (width 0.2) (layer "F.Cu") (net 17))
 (segment (start 125.074336 98.963436) (end 124.148 98.0371) (width 0.2) (layer "F.Cu") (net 17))
 (segment (start 124.148 90.89) (end 125.938 89.1) (width 0.2) (layer "F.Cu") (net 17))
 (segment (start 119.074336 101.5) (end 119.074336 57.863664) (width 0.2) (layer "F.Cu") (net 2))
 (segment (start 125.938 51) (end 127.5 51) (width 0.2) (layer "F.Cu") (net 2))
 (segment (start 119.074336 101.5) (end 116.574336 101.5) (width 0.2) (layer "F.Cu") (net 2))
 (segment (start 119.074336 57.863664) (end 125.938 51) (width 0.2) (layer "F.Cu") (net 2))
 (segment (start 123.346 98.4131) (end 123.346 86.612) (width 0.2) (layer "F.Cu") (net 15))
 (segment (start 123.346 86.612) (end 125.938 84.02) (width 0.2) (layer "F.Cu") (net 15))
 (segment (start 125.938 84.02) (end 127.5 84.02) (width 0.2) (layer "F.Cu") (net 15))
 (segment (start 124.074336 101.5) (end 124.074336 99.141436) (width 0.2) (layer "F.Cu") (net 15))
 (segment (start 124.074336 99.141436) (end 123.346 98.4131) (width 0.2) (layer "F.Cu") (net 15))
 (segment (start 125.938 81.48) (end 127.5 81.48) (width 0.2) (layer "F.Cu") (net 14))
 (segment (start 123.574336 99.208536) (end 122.945 98.5792) (width 0.2) (layer "F.Cu") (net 14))
 (segment (start 123.574336 101.5) (end 123.574336 99.208536) (width 0.2) (layer "F.Cu") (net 14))
 (segment (start 122.945 84.473) (end 125.938 81.48) (width 0.2) (layer "F.Cu") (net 14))
 (segment (start 122.945 98.5792) (end 122.945 84.473) (width 0.2) (layer "F.Cu") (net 14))
 (segment (start 124.574336 99.074336) (end 123.747 98.247) (width 0.2) (layer "F.Cu") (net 16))
 (segment (start 124.574336 101.5) (end 124.574336 99.074336) (width 0.2) (layer "F.Cu") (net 16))
 (segment (start 123.747 98.247) (end 123.747 88.751) (width 0.2) (layer "F.Cu") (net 16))
 (segment (start 125.938 86.56) (end 127.5 86.56) (width 0.2) (layer "F.Cu") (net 16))
 (segment (start 123.747 88.751) (end 125.938 86.56) (width 0.2) (layer "F.Cu") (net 16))
 (segment (start 145.28 84.02) (end 144.129 85.171) (width 0.2) (layer "F.Cu") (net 26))
 (segment (start 145.5 99.5) (end 144.129 98.129) (width 0.2) (layer "F.Cu") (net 26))
 (segment (start 144.129 85.171) (end 144.129 98.129) (width 0.2) (layer "F.Cu") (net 26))
 (segment (start 145.5 102.5) (end 145.5 99.5) (width 0.2) (layer "F.Cu") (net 26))
 (segment (start 143.5 100.5) (end 143.652 100.5) (width 0.2) (layer "F.Cu") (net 25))
 (segment (start 143.652 100.5) (end 144.5 101.348) (width 0.2) (layer "F.Cu") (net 25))
 (segment (start 143 100) (end 143.5 100.5) (width 0.2) (layer "F.Cu") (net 25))
 (segment (start 144.5 101.348) (end 144.5 102.5) (width 0.2) (layer "F.Cu") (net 25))
 (via (at 143 100) (size 0.6) (drill 0.3) (layers "F.Cu" "B.Cu") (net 25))
 (segment (start 143 100) (end 143 88.84) (width 0.2) (layer "B.Cu") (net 25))
 (segment (start 143 88.84) (end 145.28 86.56) (width 0.2) (layer "B.Cu") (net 25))
 (segment (start 145 99.5671) (end 143.728 98.2951) (width 0.2) (layer "F.Cu") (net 27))
 (segment (start 145 102.5) (end 145 99.5671) (width 0.2) (layer "F.Cu") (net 27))
 (segment (start 143.728 83.032) (end 145.28 81.48) (width 0.2) (layer "F.Cu") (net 27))
 (segment (start 143.728 98.2951) (end 143.728 83.032) (width 0.2) (layer "F.Cu") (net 27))
 (segment (start 122.544 98.7453) (end 122.544 79.794) (width 0.2) (layer "F.Cu") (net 12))
 (segment (start 123.074336 101.5) (end 123.074336 99.275636) (width 0.2) (layer "F.Cu") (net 12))
 (segment (start 125.938 76.4) (end 127.5 76.4) (width 0.2) (layer "F.Cu") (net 12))
 (segment (start 123.074336 99.275636) (end 122.544 98.7453) (width 0.2) (layer "F.Cu") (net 12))
 (segment (start 122.544 79.794) (end 125.938 76.4) (width 0.2) (layer "F.Cu") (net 12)))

